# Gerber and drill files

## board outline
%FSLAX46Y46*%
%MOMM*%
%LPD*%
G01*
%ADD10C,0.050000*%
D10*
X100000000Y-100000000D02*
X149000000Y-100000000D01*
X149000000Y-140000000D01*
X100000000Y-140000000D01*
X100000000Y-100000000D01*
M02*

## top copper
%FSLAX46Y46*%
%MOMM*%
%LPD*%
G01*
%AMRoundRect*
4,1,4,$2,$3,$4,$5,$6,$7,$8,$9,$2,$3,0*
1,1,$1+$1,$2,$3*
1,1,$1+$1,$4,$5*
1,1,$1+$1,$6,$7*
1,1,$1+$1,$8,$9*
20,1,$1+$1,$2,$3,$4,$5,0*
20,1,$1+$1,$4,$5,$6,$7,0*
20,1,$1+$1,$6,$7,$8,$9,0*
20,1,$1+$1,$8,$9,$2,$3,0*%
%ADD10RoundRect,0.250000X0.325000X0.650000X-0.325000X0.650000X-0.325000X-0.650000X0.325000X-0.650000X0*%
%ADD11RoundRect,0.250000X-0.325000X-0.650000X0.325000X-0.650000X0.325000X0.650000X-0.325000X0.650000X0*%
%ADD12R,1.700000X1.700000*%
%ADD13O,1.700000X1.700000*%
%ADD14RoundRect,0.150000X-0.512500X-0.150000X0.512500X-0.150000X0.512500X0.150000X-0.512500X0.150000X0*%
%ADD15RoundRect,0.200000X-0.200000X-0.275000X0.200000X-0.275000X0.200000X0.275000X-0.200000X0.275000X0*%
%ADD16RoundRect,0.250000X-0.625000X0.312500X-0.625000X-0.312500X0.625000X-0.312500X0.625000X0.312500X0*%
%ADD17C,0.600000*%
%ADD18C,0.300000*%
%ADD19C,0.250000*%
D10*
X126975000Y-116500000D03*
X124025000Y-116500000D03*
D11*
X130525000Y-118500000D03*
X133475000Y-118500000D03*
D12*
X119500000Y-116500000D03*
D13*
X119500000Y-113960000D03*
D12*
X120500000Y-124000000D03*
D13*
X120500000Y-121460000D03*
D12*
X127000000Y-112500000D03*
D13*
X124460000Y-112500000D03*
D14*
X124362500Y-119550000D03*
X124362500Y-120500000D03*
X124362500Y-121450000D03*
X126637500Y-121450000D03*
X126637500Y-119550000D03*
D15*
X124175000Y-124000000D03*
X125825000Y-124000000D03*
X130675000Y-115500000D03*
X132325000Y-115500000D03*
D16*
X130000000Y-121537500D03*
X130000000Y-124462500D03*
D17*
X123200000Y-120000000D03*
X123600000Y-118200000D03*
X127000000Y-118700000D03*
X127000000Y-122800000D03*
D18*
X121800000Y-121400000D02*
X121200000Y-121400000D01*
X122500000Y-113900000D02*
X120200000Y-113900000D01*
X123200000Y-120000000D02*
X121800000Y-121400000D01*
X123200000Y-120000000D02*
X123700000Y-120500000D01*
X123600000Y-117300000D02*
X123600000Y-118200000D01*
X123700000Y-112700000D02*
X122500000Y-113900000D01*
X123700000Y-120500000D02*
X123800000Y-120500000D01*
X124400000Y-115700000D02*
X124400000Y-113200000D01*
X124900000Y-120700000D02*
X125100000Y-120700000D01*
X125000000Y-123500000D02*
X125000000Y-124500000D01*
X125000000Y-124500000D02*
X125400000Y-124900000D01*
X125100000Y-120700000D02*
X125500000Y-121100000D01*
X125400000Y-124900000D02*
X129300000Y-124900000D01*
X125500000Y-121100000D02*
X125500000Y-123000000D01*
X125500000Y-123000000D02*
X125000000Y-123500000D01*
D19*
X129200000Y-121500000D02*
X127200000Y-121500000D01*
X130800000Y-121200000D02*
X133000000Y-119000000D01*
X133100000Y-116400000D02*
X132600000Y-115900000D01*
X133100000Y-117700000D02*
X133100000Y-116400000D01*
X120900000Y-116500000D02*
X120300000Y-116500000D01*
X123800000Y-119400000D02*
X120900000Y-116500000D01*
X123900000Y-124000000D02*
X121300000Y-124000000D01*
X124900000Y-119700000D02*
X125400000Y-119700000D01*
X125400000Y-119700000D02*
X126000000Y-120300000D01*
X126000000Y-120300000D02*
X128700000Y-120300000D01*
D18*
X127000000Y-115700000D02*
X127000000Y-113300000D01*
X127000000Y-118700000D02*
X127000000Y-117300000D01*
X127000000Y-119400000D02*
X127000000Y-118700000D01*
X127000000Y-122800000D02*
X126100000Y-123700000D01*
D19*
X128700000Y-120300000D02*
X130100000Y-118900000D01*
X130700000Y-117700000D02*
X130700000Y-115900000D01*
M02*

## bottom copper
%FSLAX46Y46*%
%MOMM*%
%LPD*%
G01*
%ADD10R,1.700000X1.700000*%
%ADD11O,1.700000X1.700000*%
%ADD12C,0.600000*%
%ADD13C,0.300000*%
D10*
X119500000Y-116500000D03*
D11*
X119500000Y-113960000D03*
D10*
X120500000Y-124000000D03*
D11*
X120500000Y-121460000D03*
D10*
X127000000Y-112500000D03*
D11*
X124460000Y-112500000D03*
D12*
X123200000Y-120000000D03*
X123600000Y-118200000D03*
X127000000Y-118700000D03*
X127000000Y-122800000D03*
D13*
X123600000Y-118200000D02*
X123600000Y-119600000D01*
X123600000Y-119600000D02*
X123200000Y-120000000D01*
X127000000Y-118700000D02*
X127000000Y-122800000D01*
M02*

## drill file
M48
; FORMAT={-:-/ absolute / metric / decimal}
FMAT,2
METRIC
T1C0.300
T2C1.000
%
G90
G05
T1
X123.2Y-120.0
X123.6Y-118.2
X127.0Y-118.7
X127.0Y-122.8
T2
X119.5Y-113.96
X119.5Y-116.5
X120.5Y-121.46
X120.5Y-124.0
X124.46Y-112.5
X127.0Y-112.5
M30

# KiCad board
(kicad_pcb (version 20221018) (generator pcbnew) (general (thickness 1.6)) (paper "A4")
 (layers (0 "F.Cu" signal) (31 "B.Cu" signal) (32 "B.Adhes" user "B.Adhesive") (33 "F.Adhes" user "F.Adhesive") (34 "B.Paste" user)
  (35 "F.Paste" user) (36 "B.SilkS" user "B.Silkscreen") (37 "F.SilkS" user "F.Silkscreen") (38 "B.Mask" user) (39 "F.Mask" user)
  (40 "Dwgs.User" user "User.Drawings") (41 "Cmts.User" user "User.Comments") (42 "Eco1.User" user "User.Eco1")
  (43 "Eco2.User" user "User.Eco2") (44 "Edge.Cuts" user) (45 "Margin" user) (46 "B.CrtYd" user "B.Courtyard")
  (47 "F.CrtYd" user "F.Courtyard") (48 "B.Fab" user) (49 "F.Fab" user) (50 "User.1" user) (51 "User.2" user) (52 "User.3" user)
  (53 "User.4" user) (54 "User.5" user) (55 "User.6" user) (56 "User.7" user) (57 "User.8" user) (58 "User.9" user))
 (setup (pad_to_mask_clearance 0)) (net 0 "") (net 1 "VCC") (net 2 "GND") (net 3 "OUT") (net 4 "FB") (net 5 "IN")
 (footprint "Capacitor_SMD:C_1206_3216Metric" (layer "F.Cu") (at 125.5 116.5 180)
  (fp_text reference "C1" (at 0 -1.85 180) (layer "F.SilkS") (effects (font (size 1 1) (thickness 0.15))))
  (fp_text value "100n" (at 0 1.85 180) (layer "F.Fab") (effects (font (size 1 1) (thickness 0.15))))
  (pad "1" smd roundrect (at -1.475 0 180) (size 1.15 1.8) (layers "F.Cu" "F.Paste" "F.Mask") (roundrect_rratio 0.217391) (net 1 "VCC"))
  (pad "2" smd roundrect (at 1.475 0 180) (size 1.15 1.8) (layers "F.Cu" "F.Paste" "F.Mask") (roundrect_rratio 0.217391) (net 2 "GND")))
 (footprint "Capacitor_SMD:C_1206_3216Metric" (layer "F.Cu") (at 132 118.5)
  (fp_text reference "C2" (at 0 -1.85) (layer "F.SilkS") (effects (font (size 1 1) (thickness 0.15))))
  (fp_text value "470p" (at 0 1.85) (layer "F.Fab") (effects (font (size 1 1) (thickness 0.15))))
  (pad "1" smd roundrect (at -1.475 0) (size 1.15 1.8) (layers "F.Cu" "F.Paste" "F.Mask") (roundrect_rratio 0.217391) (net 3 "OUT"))
  (pad "2" smd roundrect (at 1.475 0) (size 1.15 1.8) (layers "F.Cu" "F.Paste" "F.Mask") (roundrect_rratio 0.217391) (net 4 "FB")))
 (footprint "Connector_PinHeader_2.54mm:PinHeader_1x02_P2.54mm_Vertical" (layer "F.Cu") (at 119.5 116.5 180)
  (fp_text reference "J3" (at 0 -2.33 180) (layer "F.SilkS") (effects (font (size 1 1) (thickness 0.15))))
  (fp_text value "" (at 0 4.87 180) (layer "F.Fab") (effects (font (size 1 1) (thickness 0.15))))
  (pad "1" thru_hole rect (at 0 0 180) (size 1.7 1.7) (drill 1) (layers "*.Cu" "*.Mask") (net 3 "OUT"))
  (pad "2" thru_hole oval (at 0 2.54 180) (size 1.7 1.7) (drill 1) (layers "*.Cu" "*.Mask") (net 2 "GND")))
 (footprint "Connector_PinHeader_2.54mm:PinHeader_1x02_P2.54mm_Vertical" (layer "F.Cu") (at 120.5 124 180)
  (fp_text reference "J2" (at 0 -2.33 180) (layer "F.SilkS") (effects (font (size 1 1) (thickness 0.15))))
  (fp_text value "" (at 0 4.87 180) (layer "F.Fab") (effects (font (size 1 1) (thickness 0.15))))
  (pad "1" thru_hole rect (at 0 0 180) (size 1.7 1.7) (drill 1) (layers "*.Cu" "*.Mask") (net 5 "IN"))
  (pad "2" thru_hole oval (at 0 2.54 180) (size 1.7 1.7) (drill 1) (layers "*.Cu" "*.Mask") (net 2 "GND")))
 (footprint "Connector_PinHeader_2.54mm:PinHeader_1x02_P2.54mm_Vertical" (layer "F.Cu") (at 127 112.5 -90)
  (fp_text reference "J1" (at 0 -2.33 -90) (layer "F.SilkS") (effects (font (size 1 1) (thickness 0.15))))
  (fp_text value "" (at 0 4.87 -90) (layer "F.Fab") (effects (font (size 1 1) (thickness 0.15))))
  (pad "1" thru_hole rect (at 0 0 270) (size 1.7 1.7) (drill 1) (layers "*.Cu" "*.Mask") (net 1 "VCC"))
  (pad "2" thru_hole oval (at 0 2.54 270) (size 1.7 1.7) (drill 1) (layers "*.Cu" "*.Mask") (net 2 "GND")))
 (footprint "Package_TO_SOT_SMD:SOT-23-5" (layer "F.Cu") (at 125.5 120.5)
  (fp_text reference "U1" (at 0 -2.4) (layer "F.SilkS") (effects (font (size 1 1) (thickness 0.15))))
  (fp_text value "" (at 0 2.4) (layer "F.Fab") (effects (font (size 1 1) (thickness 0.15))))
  (pad "1" smd roundrect (at -1.1375 -0.95) (size 1.325 0.6) (layers "F.Cu" "F.Paste" "F.Mask") (roundrect_rratio 0.25) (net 3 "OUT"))
  (pad "2" smd roundrect (at -1.1375 0) (size 1.325 0.6) (layers "F.Cu" "F.Paste" "F.Mask") (roundrect_rratio 0.25) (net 2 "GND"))
  (pad "3" smd roundrect (at -1.1375 0.95) (size 1.325 0.6) (layers "F.Cu" "F.Paste" "F.Mask") (roundrect_rratio 0.25))
  (pad "4" smd roundrect (at 1.1375 0.95) (size 1.325 0.6) (layers "F.Cu" "F.Paste" "F.Mask") (roundrect_rratio 0.25) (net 4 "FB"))
  (pad "5" smd roundrect (at 1.1375 -0.95) (size 1.325 0.6) (layers "F.Cu" "F.Paste" "F.Mask") (roundrect_rratio 0.25) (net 1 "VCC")))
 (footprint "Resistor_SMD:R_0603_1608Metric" (layer "F.Cu") (at 125 124)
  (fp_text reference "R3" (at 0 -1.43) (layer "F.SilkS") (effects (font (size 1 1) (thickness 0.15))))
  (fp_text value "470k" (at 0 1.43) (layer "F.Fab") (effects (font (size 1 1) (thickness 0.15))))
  (pad "1" smd roundrect (at -0.825 0) (size 0.8 0.95) (layers "F.Cu" "F.Paste" "F.Mask") (roundrect_rratio 0.25) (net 5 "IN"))
  (pad "2" smd roundrect (at 0.825 0) (size 0.8 0.95) (layers "F.Cu" "F.Paste" "F.Mask") (roundrect_rratio 0.25) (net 1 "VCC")))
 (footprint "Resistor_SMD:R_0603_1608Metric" (layer "F.Cu") (at 131.5 115.5)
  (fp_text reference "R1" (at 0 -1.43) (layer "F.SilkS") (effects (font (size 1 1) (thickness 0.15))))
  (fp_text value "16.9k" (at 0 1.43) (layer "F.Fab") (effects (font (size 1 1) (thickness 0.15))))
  (pad "1" smd roundrect (at -0.825 0) (size 0.8 0.95) (layers "F.Cu" "F.Paste" "F.Mask") (roundrect_rratio 0.25) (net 3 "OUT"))
  (pad "2" smd roundrect (at 0.825 0) (size 0.8 0.95) (layers "F.Cu" "F.Paste" "F.Mask") (roundrect_rratio 0.25) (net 4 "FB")))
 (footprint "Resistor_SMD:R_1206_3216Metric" (layer "F.Cu") (at 130 123 -90)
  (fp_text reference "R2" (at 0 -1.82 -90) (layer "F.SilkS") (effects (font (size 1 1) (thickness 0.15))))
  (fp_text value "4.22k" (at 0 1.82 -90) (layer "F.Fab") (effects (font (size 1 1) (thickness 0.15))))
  (pad "1" smd roundrect (at -1.4625 0 270) (size 1.125 1.75) (layers "F.Cu" "F.Paste" "F.Mask") (roundrect_rratio 0.222222) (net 4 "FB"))
  (pad "2" smd roundrect (at 1.4625 0 270) (size 1.125 1.75) (layers "F.Cu" "F.Paste" "F.Mask") (roundrect_rratio 0.222222) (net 2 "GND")))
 (gr_rect (start 100 100) (end 149 140) (stroke (width 0.05) (type default)) (fill none) (layer "Edge.Cuts"))
 (segment (start 121.8 121.4) (end 121.2 121.4) (width 0.3) (layer "F.Cu") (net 2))
 (segment (start 122.5 113.9) (end 120.2 113.9) (width 0.3) (layer "F.Cu") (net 2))
 (segment (start 123.2 120) (end 121.8 121.4) (width 0.3) (layer "F.Cu") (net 2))
 (segment (start 123.2 120) (end 123.7 120.5) (width 0.3) (layer "F.Cu") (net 2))
 (segment (start 123.6 117.3) (end 123.6 118.2) (width 0.3) (layer "F.Cu") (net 2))
 (segment (start 123.7 112.7) (end 122.5 113.9) (width 0.3) (layer "F.Cu") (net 2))
 (segment (start 123.7 120.5) (end 123.8 120.5) (width 0.3) (layer "F.Cu") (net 2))
 (segment (start 124.4 115.7) (end 124.4 113.2) (width 0.3) (layer "F.Cu") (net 2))
 (segment (start 124.9 120.7) (end 125.1 120.7) (width 0.3) (layer "F.Cu") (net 2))
 (segment (start 125 123.5) (end 125 124.5) (width 0.3) (layer "F.Cu") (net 2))
 (segment (start 125 124.5) (end 125.4 124.9) (width 0.3) (layer "F.Cu") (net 2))
 (segment (start 125.1 120.7) (end 125.5 121.1) (width 0.3) (layer "F.Cu") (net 2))
 (segment (start 125.4 124.9) (end 129.3 124.9) (width 0.3) (layer "F.Cu") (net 2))
 (segment (start 125.5 121.1) (end 125.5 123) (width 0.3) (layer "F.Cu") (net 2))
 (segment (start 125.5 123) (end 125 123.5) (width 0.3) (layer "F.Cu") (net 2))
 (segment (start 129.2 121.5) (end 127.2 121.5) (width 0.25) (layer "F.Cu") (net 4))
 (segment (start 130.8 121.2) (end 133 119) (width 0.25) (layer "F.Cu") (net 4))
 (segment (start 133.1 116.4) (end 132.6 115.9) (width 0.25) (layer "F.Cu") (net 4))
 (segment (start 133.1 117.7) (end 133.1 116.4) (width 0.25) (layer "F.Cu") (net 4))
 (via (at 123.2 120) (size 0.6) (drill 0.3) (layers "F.Cu" "B.Cu") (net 2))
 (via (at 123.6 118.2) (size 0.6) (drill 0.3) (layers "F.Cu" "B.Cu") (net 2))
 (segment (start 120.9 116.5) (end 120.3 116.5) (width 0.25) (layer "F.Cu") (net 3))
 (segment (start 123.6 118.2) (end 123.6 119.6) (width 0.3) (layer "B.Cu") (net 2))
 (segment (start 123.6 119.6) (end 123.2 120) (width 0.3) (layer "B.Cu") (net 2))
 (segment (start 123.8 119.4) (end 120.9 116.5) (width 0.25) (layer "F.Cu") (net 3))
 (segment (start 123.9 124) (end 121.3 124) (width 0.25) (layer "F.Cu") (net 5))
 (segment (start 124.9 119.7) (end 125.4 119.7) (width 0.25) (layer "F.Cu") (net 3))
 (segment (start 125.4 119.7) (end 126 120.3) (width 0.25) (layer "F.Cu") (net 3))
 (segment (start 126 120.3) (end 128.7 120.3) (width 0.25) (layer "F.Cu") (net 3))
 (segment (start 127 115.7) (end 127 113.3) (width 0.3) (layer "F.Cu") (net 1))
 (segment (start 127 118.7) (end 127 117.3) (width 0.3) (layer "F.Cu") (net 1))
 (segment (start 127 119.4) (end 127 118.7) (width 0.3) (layer "F.Cu") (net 1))
 (segment (start 127 122.8) (end 126.1 123.7) (width 0.3) (layer "F.Cu") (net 1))
 (segment (start 128.7 120.3) (end 130.1 118.9) (width 0.25) (layer "F.Cu") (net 3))
 (segment (start 130.7 117.7) (end 130.7 115.9) (width 0.25) (layer "F.Cu") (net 3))
 (via (at 127 118.7) (size 0.6) (drill 0.3) (layers "F.Cu" "B.Cu") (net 1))
 (via (at 127 122.8) (size 0.6) (drill 0.3) (layers "F.Cu" "B.Cu") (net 1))
 (segment (start 127 118.7) (end 127 122.8) (width 0.3) (layer "B.Cu") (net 1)))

